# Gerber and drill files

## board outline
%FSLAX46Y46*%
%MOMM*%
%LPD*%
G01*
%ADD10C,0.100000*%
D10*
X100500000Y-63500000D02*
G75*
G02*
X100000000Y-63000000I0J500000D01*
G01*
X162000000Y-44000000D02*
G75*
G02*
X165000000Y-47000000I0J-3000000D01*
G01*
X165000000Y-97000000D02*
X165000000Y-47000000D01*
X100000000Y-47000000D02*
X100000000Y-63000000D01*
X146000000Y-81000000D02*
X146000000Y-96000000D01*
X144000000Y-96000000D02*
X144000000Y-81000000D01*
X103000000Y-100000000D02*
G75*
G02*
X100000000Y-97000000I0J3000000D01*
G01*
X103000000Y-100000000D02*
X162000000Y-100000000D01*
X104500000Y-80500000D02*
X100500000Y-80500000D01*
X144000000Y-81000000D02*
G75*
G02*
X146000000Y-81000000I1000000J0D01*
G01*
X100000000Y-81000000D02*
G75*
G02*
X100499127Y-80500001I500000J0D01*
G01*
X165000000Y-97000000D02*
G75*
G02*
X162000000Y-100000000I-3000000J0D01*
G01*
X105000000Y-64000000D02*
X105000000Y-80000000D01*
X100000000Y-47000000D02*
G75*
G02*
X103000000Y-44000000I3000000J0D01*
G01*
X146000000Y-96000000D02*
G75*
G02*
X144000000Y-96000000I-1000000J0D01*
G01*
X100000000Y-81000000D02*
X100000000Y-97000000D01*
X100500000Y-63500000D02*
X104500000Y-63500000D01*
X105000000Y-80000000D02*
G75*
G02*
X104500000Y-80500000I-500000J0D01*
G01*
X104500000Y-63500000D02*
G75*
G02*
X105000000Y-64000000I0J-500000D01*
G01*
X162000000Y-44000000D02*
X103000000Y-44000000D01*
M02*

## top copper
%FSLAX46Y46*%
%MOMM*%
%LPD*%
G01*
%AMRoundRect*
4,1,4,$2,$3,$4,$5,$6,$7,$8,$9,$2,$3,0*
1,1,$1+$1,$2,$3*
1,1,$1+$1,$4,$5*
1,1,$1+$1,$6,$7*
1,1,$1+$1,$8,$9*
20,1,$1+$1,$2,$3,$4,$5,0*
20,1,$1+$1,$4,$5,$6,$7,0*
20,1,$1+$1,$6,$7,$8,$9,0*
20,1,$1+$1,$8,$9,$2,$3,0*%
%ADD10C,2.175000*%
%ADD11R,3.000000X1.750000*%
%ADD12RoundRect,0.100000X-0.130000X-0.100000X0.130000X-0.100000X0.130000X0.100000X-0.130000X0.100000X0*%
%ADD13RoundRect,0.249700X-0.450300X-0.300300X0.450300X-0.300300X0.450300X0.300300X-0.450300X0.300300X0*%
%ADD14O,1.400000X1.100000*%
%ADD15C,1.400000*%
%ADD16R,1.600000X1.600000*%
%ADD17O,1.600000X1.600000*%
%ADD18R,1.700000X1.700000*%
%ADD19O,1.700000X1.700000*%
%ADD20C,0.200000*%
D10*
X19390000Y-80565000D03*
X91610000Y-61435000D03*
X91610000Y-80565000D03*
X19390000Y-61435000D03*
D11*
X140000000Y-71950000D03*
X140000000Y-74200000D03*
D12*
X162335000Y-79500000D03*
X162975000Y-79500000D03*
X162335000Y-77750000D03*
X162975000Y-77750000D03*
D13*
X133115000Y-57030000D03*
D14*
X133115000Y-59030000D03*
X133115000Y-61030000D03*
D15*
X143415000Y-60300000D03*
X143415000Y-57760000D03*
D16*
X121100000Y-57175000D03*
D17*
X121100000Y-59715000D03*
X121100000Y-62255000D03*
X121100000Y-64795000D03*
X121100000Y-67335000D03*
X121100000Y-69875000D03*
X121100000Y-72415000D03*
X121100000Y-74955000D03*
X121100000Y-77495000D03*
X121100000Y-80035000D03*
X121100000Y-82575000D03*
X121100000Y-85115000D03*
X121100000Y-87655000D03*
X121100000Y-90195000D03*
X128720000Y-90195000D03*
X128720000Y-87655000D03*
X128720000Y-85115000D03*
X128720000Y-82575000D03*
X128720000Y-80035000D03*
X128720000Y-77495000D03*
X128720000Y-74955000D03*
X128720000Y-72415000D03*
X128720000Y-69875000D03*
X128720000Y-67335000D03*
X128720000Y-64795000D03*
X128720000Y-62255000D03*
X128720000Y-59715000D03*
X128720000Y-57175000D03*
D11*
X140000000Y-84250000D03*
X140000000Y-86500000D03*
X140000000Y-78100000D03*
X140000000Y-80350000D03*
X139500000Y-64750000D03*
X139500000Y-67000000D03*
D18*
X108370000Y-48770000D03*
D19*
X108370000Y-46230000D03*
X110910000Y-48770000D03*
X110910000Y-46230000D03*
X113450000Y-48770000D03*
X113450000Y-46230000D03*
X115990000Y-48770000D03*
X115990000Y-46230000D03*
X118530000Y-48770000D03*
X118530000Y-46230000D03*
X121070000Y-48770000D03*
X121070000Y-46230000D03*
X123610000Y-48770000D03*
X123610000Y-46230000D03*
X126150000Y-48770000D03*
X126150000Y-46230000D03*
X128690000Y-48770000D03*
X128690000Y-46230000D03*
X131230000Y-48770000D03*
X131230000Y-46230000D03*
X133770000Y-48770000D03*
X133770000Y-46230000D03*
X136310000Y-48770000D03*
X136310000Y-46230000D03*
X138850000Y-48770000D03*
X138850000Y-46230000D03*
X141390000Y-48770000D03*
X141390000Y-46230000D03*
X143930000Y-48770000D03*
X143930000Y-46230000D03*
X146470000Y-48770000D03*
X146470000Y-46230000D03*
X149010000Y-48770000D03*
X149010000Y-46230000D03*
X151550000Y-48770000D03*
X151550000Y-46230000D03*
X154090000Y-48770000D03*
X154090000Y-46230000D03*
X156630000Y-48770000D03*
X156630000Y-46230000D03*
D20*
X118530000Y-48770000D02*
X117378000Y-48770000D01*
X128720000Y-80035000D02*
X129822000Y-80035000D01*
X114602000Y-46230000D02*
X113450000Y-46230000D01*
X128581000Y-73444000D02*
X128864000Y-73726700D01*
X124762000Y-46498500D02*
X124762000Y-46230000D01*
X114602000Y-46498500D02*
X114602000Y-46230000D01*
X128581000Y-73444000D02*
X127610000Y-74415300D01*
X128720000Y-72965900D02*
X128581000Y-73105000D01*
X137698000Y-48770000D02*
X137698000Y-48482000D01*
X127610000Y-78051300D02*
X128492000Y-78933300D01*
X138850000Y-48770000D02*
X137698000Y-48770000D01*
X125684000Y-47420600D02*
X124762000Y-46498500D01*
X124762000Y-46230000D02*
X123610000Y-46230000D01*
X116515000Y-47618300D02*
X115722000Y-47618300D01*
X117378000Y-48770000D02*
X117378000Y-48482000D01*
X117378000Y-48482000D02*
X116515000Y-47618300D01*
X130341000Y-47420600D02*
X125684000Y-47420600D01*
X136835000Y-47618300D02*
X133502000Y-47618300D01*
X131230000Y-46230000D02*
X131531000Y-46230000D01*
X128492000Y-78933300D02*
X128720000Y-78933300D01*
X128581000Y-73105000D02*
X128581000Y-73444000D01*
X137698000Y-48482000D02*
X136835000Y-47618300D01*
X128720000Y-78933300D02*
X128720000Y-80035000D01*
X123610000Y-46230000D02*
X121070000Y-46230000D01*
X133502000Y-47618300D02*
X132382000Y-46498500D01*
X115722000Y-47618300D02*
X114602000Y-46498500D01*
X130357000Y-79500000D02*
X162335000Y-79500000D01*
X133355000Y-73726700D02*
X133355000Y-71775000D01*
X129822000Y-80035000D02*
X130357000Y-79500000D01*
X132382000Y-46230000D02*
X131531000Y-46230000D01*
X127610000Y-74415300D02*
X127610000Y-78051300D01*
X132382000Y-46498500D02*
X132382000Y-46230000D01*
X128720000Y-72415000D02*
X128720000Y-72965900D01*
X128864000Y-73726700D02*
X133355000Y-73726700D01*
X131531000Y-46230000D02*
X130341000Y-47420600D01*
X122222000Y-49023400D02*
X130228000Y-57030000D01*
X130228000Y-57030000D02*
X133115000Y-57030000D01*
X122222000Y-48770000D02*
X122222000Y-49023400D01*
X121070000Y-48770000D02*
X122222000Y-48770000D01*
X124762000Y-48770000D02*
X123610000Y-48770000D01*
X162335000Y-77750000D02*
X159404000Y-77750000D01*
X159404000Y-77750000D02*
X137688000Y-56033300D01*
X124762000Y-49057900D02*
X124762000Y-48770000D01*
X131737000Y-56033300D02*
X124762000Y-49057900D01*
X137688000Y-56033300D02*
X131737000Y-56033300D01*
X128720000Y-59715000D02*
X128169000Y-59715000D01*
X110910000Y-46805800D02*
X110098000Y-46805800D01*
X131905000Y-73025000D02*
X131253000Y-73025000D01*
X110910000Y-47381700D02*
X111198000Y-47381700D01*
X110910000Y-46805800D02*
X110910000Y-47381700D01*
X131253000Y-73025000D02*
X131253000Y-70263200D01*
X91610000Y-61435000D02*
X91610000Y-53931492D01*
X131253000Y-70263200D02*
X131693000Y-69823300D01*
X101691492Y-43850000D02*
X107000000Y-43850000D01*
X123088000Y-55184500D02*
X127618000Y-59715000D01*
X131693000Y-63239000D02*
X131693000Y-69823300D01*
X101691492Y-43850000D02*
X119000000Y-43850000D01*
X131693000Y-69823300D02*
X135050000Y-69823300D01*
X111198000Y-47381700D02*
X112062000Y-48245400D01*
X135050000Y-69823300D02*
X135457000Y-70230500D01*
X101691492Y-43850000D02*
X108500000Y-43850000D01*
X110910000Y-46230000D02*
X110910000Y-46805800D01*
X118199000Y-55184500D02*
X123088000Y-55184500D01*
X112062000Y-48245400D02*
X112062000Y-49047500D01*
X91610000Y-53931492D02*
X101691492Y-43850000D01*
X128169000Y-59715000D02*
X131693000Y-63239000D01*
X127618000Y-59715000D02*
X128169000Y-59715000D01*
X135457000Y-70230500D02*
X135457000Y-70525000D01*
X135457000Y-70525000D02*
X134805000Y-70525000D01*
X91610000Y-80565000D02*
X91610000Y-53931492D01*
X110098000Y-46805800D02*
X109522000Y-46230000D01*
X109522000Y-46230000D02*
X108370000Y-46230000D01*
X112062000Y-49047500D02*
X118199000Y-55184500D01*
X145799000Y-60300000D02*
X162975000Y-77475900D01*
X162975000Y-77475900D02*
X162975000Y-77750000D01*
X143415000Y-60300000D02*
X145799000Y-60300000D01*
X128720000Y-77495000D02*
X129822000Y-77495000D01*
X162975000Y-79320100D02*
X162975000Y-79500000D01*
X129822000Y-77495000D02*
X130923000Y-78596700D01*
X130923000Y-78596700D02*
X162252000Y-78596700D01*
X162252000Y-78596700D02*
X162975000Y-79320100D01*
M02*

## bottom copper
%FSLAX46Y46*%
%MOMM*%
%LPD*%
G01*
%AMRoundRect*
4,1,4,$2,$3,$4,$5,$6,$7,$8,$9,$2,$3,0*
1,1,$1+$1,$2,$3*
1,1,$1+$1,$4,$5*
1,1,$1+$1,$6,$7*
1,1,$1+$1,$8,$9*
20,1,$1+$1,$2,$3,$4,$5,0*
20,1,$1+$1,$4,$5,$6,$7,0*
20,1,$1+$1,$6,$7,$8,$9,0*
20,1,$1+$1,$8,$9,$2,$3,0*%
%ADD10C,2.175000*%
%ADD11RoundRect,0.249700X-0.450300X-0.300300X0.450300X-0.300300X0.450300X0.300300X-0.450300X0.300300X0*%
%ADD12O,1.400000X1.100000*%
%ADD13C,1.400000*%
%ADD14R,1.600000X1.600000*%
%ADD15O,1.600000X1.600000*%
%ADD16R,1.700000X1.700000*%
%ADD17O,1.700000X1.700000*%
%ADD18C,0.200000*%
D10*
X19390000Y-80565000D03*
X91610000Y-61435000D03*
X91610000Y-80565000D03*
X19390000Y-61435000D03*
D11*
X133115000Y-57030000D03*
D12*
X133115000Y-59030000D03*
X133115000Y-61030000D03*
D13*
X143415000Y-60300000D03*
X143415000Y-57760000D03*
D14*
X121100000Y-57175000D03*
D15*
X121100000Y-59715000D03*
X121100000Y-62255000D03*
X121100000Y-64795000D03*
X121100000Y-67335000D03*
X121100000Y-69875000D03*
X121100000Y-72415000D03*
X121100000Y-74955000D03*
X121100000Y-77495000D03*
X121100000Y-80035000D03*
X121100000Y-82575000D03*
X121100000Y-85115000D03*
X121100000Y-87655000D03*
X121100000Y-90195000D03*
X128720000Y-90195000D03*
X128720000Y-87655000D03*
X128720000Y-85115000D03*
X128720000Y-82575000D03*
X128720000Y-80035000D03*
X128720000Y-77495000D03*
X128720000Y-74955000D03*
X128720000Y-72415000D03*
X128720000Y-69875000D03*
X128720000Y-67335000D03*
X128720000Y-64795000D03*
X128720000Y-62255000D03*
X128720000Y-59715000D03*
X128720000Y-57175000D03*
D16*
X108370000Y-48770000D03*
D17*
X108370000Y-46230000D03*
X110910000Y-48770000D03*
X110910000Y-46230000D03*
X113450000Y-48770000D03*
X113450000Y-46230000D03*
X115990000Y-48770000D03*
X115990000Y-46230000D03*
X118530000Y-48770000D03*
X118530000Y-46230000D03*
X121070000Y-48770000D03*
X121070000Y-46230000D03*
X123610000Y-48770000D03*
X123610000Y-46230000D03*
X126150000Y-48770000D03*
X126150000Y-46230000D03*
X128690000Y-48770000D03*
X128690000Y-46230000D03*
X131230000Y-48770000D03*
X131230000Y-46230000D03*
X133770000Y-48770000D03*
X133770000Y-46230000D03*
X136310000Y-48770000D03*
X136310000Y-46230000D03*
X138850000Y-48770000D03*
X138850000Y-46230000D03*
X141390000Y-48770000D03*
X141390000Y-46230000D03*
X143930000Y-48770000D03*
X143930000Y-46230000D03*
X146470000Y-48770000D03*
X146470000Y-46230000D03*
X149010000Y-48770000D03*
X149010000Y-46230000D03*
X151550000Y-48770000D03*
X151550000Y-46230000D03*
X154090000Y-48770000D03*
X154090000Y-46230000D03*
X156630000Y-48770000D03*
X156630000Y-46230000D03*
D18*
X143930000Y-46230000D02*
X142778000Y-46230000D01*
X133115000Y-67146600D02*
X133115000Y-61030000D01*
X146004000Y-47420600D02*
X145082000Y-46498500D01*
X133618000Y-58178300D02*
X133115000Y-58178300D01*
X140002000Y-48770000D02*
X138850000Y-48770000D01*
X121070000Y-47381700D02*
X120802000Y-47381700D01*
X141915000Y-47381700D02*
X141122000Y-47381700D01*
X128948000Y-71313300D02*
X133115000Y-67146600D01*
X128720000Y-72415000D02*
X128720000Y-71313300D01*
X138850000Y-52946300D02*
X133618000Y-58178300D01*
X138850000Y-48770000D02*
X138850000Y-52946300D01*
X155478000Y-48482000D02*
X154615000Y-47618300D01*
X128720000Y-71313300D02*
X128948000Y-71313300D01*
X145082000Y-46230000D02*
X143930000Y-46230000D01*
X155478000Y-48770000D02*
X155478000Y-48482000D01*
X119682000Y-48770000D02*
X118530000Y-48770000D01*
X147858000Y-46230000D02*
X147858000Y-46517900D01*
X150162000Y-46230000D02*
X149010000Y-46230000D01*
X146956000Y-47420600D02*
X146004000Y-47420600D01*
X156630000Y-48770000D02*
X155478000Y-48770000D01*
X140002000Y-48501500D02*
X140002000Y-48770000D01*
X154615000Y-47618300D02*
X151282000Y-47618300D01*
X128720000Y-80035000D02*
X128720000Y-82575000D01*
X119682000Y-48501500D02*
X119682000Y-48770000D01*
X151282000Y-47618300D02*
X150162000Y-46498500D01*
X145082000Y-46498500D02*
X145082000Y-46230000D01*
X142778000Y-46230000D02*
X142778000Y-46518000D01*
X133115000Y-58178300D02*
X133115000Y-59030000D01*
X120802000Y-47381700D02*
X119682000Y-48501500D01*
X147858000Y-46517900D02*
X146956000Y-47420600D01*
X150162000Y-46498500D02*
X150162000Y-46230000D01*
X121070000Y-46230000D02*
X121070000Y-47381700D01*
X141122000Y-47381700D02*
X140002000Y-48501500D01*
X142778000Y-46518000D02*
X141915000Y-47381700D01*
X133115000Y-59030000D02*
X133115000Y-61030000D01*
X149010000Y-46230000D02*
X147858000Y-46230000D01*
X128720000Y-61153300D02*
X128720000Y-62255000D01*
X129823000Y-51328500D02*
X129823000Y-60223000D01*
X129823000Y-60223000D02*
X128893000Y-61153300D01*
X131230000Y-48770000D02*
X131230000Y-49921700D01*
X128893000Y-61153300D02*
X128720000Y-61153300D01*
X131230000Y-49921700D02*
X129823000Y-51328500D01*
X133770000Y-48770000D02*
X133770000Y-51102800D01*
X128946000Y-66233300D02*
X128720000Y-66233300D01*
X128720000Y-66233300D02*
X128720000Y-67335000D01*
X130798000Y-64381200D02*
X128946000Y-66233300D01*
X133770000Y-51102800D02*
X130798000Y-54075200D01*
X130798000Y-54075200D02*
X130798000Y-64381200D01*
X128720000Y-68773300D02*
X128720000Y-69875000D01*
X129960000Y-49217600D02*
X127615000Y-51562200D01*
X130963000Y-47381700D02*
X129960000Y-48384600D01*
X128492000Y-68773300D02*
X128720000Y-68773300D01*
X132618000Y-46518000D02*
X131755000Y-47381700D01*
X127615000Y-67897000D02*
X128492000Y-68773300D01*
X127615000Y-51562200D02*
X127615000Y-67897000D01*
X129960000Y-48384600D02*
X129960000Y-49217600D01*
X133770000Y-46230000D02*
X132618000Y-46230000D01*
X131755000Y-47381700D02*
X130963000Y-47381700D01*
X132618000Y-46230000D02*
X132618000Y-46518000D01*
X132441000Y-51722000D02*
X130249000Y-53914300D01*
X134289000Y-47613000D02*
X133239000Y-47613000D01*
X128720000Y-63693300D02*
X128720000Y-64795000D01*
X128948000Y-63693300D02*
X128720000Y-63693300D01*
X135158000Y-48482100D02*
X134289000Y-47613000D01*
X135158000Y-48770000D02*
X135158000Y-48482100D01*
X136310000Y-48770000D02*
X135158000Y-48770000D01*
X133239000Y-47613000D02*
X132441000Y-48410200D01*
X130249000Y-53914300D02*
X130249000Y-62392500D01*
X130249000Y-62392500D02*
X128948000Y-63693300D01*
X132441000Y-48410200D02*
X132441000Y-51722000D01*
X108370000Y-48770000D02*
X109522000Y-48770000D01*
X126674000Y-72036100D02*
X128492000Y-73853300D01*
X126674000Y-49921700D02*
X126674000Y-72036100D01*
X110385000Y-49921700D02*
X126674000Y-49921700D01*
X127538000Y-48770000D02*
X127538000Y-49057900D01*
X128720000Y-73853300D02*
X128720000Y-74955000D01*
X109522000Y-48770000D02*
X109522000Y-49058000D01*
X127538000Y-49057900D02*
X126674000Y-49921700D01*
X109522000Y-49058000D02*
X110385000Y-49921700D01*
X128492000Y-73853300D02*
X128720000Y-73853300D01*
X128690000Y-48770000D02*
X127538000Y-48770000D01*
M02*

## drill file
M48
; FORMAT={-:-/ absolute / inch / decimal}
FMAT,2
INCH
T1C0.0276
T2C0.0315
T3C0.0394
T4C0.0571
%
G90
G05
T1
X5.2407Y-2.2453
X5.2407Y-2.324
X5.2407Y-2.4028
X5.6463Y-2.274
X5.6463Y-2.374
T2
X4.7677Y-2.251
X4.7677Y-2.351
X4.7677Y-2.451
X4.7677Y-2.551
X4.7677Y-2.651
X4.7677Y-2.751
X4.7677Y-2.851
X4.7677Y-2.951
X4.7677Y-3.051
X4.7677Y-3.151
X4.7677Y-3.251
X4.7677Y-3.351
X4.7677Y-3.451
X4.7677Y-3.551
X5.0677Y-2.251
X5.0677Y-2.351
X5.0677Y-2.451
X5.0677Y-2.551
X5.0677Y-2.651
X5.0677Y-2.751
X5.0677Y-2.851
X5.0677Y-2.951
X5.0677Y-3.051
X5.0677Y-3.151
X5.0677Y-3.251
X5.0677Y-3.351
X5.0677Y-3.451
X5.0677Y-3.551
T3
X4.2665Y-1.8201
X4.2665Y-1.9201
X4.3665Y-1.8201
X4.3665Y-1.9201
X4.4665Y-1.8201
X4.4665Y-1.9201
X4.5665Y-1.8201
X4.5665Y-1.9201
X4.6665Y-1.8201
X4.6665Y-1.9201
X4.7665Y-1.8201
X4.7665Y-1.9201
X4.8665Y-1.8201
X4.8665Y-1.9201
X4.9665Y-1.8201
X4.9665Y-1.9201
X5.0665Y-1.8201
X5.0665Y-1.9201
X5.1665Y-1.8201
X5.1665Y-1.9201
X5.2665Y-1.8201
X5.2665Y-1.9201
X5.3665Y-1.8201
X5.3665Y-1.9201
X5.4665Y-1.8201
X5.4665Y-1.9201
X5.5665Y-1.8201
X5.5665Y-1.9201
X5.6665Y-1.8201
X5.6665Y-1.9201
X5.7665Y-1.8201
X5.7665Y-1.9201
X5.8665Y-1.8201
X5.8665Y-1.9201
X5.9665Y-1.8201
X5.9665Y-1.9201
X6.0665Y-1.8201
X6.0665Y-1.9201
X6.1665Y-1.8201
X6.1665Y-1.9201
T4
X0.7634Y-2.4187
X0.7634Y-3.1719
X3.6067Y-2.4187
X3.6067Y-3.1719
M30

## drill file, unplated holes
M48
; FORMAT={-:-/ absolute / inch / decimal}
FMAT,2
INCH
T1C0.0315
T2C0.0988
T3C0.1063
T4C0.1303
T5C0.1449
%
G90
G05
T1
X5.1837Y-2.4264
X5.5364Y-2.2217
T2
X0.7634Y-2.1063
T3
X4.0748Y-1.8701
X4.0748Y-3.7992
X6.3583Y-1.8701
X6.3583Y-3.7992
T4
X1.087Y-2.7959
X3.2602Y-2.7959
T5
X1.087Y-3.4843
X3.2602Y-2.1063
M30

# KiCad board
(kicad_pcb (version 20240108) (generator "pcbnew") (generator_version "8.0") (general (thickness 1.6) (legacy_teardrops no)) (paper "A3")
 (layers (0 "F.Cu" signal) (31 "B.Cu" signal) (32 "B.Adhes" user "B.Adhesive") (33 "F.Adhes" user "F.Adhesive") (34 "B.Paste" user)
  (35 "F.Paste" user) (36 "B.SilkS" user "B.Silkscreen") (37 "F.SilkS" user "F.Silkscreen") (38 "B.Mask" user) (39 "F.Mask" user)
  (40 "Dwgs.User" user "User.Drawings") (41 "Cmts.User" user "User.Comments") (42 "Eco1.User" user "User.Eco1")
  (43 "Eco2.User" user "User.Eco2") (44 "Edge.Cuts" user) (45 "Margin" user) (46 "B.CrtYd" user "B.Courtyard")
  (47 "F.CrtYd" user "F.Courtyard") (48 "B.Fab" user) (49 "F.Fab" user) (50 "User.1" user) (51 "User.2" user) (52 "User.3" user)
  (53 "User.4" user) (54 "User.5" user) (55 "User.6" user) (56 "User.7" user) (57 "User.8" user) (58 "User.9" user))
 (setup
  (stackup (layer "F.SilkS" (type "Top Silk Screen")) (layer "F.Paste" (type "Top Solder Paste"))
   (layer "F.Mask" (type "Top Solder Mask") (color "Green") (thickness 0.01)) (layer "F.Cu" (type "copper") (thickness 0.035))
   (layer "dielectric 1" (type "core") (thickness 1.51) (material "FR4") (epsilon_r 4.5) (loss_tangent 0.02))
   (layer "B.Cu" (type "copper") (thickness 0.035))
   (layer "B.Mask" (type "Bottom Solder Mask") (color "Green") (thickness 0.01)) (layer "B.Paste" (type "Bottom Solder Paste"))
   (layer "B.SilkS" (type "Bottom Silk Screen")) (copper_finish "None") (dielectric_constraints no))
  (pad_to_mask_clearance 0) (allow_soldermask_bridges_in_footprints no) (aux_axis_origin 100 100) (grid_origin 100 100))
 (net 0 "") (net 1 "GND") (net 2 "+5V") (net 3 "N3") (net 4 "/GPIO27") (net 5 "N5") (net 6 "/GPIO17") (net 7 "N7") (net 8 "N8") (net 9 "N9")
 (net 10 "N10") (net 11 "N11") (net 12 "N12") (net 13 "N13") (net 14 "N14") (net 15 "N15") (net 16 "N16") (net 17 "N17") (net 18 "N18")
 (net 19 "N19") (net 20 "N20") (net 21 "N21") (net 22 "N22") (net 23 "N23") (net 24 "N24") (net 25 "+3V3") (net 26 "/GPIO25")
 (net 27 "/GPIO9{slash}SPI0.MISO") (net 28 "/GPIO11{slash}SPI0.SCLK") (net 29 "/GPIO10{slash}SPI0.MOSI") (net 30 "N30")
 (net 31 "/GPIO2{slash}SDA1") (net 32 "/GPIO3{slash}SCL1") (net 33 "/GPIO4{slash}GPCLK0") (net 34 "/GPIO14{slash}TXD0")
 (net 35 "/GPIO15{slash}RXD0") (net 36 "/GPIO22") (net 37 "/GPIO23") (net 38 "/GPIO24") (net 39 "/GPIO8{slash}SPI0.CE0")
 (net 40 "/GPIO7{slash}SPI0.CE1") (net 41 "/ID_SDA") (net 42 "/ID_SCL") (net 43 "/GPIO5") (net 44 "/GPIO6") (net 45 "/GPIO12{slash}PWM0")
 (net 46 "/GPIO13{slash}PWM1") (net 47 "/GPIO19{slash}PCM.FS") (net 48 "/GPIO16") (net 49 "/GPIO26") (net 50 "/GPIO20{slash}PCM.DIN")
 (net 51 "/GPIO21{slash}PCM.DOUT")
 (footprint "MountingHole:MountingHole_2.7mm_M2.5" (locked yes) (layer "F.Cu") (at 161.5 47.5)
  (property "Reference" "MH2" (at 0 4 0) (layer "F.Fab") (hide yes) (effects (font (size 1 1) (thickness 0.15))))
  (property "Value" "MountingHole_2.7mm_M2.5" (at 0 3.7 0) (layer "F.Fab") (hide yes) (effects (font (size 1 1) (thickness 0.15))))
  (pad "" np_thru_hole circle (at 0 0) (size 2.7 2.7) (drill 2.7) (layers "*.Cu" "*.Mask")))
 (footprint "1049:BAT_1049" (layer "F.Cu") (at 55.5 71 180)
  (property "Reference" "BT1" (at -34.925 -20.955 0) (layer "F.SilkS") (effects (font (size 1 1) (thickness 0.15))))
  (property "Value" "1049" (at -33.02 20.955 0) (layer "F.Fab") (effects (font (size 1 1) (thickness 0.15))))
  (pad "" np_thru_hole circle (at -27.31 -0.015 180) (size 3.31 3.31) (drill 3.31) (layers "*.Cu" "*.Mask"))
  (pad "" np_thru_hole circle (at -27.31 17.5 180) (size 3.68 3.68) (drill 3.68) (layers "*.Cu" "*.Mask"))
  (pad "" np_thru_hole circle (at 27.89 -17.5 180) (size 3.68 3.68) (drill 3.68) (layers "*.Cu" "*.Mask"))
  (pad "" np_thru_hole circle (at 27.89 -0.015 180) (size 3.31 3.31) (drill 3.31) (layers "*.Cu" "*.Mask"))
  (pad "" np_thru_hole circle (at 36.11 17.5 180) (size 2.51 2.51) (drill 2.51) (layers "*.Cu" "*.Mask"))
  (pad "N1" thru_hole circle (at 36.11 -9.565 180) (size 2.175 2.175) (drill 1.45) (layers "*.Cu" "*.Mask") (remove_unused_layers no)
   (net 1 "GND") (solder_mask_margin 0.102))
  (pad "N2" thru_hole circle (at -36.11 9.565 180) (size 2.175 2.175) (drill 1.45) (layers "*.Cu" "*.Mask") (remove_unused_layers no)
   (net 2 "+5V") (solder_mask_margin 0.102))
  (pad "P1" thru_hole circle (at -36.11 -9.565 180) (size 2.175 2.175) (drill 1.45) (layers "*.Cu" "*.Mask") (remove_unused_layers no)
   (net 2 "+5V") (solder_mask_margin 0.102))
  (pad "P2" thru_hole circle (at 36.11 9.565 180) (size 2.175 2.175) (drill 1.45) (layers "*.Cu" "*.Mask") (remove_unused_layers no)
   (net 1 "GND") (solder_mask_margin 0.102)))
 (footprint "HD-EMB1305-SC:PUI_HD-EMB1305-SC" (layer "F.Cu") (at 140 73.075)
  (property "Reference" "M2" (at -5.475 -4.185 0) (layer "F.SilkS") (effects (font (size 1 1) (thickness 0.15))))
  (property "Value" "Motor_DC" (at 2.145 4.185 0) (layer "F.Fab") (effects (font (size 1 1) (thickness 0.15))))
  (pad "N" smd rect (at 0 -1.125) (size 3 1.75) (layers "F.Cu" "F.Paste" "F.Mask") (solder_mask_margin 0.102))
  (pad "P" smd rect (at 0 1.125) (size 3 1.75) (layers "F.Cu" "F.Paste" "F.Mask") (solder_mask_margin 0.102)))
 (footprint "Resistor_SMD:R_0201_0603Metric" (layer "F.Cu") (at 162.655 79.5)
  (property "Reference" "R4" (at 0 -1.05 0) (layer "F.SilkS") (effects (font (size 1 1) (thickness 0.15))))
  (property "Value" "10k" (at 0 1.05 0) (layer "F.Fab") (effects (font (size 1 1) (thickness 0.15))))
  (pad "" smd roundrect (at -0.345 0) (size 0.318 0.36) (layers "F.Paste") (roundrect_rratio 0.25))
  (pad "" smd roundrect (at 0.345 0) (size 0.318 0.36) (layers "F.Paste") (roundrect_rratio 0.25))
  (pad "1" smd roundrect (at -0.32 0) (size 0.46 0.4) (layers "F.Cu" "F.Mask") (roundrect_rratio 0.25) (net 1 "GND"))
  (pad "2" smd roundrect (at 0.32 0) (size 0.46 0.4) (layers "F.Cu" "F.Mask") (roundrect_rratio 0.25) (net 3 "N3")))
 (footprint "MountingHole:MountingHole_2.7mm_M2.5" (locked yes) (layer "F.Cu") (at 103.5 96.5)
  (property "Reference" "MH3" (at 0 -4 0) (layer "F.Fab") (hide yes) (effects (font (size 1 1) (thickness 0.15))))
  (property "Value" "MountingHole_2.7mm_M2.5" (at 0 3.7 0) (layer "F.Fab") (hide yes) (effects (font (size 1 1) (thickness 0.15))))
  (pad "" np_thru_hole circle (at 0 0) (size 2.7 2.7) (drill 2.7) (layers "*.Cu" "*.Mask")))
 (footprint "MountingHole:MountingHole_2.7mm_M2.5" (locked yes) (layer "F.Cu") (at 103.5 47.5)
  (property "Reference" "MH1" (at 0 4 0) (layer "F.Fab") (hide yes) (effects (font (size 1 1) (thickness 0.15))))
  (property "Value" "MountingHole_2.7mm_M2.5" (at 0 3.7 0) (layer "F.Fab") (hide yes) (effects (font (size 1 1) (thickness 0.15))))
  (pad "" np_thru_hole circle (at 0 0) (size 2.7 2.7) (drill 2.7) (layers "*.Cu" "*.Mask")))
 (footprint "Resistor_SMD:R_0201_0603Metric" (layer "F.Cu") (at 162.655 77.75)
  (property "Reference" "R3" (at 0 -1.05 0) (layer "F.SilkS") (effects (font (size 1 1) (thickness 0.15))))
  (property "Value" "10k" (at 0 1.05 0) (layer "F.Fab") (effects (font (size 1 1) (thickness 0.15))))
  (pad "" smd roundrect (at -0.345 0) (size 0.318 0.36) (layers "F.Paste") (roundrect_rratio 0.25))
  (pad "" smd roundrect (at 0.345 0) (size 0.318 0.36) (layers "F.Paste") (roundrect_rratio 0.25))
  (pad "1" smd roundrect (at -0.32 0) (size 0.46 0.4) (layers "F.Cu" "F.Mask") (roundrect_rratio 0.25) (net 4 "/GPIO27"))
  (pad "2" smd roundrect (at 0.32 0) (size 0.46 0.4) (layers "F.Cu" "F.Mask") (roundrect_rratio 0.25) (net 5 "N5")))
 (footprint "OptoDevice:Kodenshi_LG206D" (layer "F.Cu") (at 133.115 57.03)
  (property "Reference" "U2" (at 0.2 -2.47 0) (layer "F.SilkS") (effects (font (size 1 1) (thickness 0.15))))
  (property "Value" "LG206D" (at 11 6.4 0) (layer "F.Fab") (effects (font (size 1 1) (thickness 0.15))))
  (pad "" np_thru_hole circle (at -1.45 4.6) (size 0.8 0.8) (drill 0.8) (layers "*.Cu" "*.Mask"))
  (pad "" np_thru_hole circle (at 7.51 -0.6) (size 0.8 0.8) (drill 0.8) (layers "*.Cu" "*.Mask"))
  (pad "1" thru_hole roundrect (at 0 0) (size 1.4 1.1) (drill 0.7) (layers "*.Cu" "*.Mask") (remove_unused_layers no)
   (roundrect_rratio 0.227) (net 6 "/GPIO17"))
  (pad "2" thru_hole oval (at 0 2) (size 1.4 1.1) (drill 0.7) (layers "*.Cu" "*.Mask") (remove_unused_layers no) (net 1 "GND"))
  (pad "3" thru_hole oval (at 0 4) (size 1.4 1.1) (drill 0.7) (layers "*.Cu" "*.Mask") (remove_unused_layers no) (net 1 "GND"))
  (pad "4" thru_hole circle (at 10.3 3.27) (size 1.4 1.4) (drill 0.7) (layers "*.Cu" "*.Mask") (remove_unused_layers no) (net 5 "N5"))
  (pad "5" thru_hole circle (at 10.3 0.73) (size 1.4 1.4) (drill 0.7) (layers "*.Cu" "*.Mask") (remove_unused_layers no) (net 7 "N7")))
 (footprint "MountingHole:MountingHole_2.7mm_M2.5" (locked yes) (layer "F.Cu") (at 161.5 96.5)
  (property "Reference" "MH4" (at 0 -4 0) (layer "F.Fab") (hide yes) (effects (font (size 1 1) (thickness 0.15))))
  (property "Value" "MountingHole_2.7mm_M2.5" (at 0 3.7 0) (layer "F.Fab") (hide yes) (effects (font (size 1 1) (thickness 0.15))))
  (pad "" np_thru_hole circle (at 0 0) (size 2.7 2.7) (drill 2.7) (layers "*.Cu" "*.Mask")))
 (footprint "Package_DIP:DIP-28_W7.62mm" (layer "F.Cu") (at 121.1 57.175)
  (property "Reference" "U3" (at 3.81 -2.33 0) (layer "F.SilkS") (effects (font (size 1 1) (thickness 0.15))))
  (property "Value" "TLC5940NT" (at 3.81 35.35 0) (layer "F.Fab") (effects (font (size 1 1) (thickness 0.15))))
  (pad "1" thru_hole rect (at 0 0) (size 1.6 1.6) (drill 0.8) (layers "*.Cu" "*.Mask") (remove_unused_layers no) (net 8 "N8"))
  (pad "2" thru_hole oval (at 0 2.54) (size 1.6 1.6) (drill 0.8) (layers "*.Cu" "*.Mask") (remove_unused_layers no) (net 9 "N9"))
  (pad "3" thru_hole oval (at 0 5.08) (size 1.6 1.6) (drill 0.8) (layers "*.Cu" "*.Mask") (remove_unused_layers no) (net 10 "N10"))
  (pad "4" thru_hole oval (at 0 7.62) (size 1.6 1.6) (drill 0.8) (layers "*.Cu" "*.Mask") (remove_unused_layers no) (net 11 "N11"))
  (pad "5" thru_hole oval (at 0 10.16) (size 1.6 1.6) (drill 0.8) (layers "*.Cu" "*.Mask") (remove_unused_layers no) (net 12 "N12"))
  (pad "6" thru_hole oval (at 0 12.7) (size 1.6 1.6) (drill 0.8) (layers "*.Cu" "*.Mask") (remove_unused_layers no) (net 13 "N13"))
  (pad "7" thru_hole oval (at 0 15.24) (size 1.6 1.6) (drill 0.8) (layers "*.Cu" "*.Mask") (remove_unused_layers no) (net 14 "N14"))
  (pad "8" thru_hole oval (at 0 17.78) (size 1.6 1.6) (drill 0.8) (layers "*.Cu" "*.Mask") (remove_unused_layers no) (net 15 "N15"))
  (pad "9" thru_hole oval (at 0 20.32) (size 1.6 1.6) (drill 0.8) (layers "*.Cu" "*.Mask") (remove_unused_layers no) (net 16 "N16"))
  (pad "10" thru_hole oval (at 0 22.86) (size 1.6 1.6) (drill 0.8) (layers "*.Cu" "*.Mask") (remove_unused_layers no) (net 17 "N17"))
  (pad "11" thru_hole oval (at 0 25.4) (size 1.6 1.6) (drill 0.8) (layers "*.Cu" "*.Mask") (remove_unused_layers no) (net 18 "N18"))
  (pad "12" thru_hole oval (at 0 27.94) (size 1.6 1.6) (drill 0.8) (layers "*.Cu" "*.Mask") (remove_unused_layers no) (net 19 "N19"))
  (pad "13" thru_hole oval (at 0 30.48) (size 1.6 1.6) (drill 0.8) (layers "*.Cu" "*.Mask") (remove_unused_layers no) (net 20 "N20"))
  (pad "14" thru_hole oval (at 0 33.02) (size 1.6 1.6) (drill 0.8) (layers "*.Cu" "*.Mask") (remove_unused_layers no) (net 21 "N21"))
  (pad "15" thru_hole oval (at 7.62 33.02) (size 1.6 1.6) (drill 0.8) (layers "*.Cu" "*.Mask") (remove_unused_layers no) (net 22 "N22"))
  (pad "16" thru_hole oval (at 7.62 30.48) (size 1.6 1.6) (drill 0.8) (layers "*.Cu" "*.Mask") (remove_unused_layers no) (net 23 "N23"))
  (pad "17" thru_hole oval (at 7.62 27.94) (size 1.6 1.6) (drill 0.8) (layers "*.Cu" "*.Mask") (remove_unused_layers no) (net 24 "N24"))
  (pad "18" thru_hole oval (at 7.62 25.4) (size 1.6 1.6) (drill 0.8) (layers "*.Cu" "*.Mask") (remove_unused_layers no) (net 1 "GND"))
  (pad "19" thru_hole oval (at 7.62 22.86) (size 1.6 1.6) (drill 0.8) (layers "*.Cu" "*.Mask") (remove_unused_layers no) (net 1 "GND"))
  (pad "20" thru_hole oval (at 7.62 20.32) (size 1.6 1.6) (drill 0.8) (layers "*.Cu" "*.Mask") (remove_unused_layers no) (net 3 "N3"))
  (pad "21" thru_hole oval (at 7.62 17.78) (size 1.6 1.6) (drill 0.8) (layers "*.Cu" "*.Mask") (remove_unused_layers no) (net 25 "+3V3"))
  (pad "22" thru_hole oval (at 7.62 15.24) (size 1.6 1.6) (drill 0.8) (layers "*.Cu" "*.Mask") (remove_unused_layers no) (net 1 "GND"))
  (pad "23" thru_hole oval (at 7.62 12.7) (size 1.6 1.6) (drill 0.8) (layers "*.Cu" "*.Mask") (remove_unused_layers no) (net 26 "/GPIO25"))
  (pad "24" thru_hole oval (at 7.62 10.16) (size 1.6 1.6) (drill 0.8) (layers "*.Cu" "*.Mask") (remove_unused_layers no)
   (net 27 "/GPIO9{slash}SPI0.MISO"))
  (pad "25" thru_hole oval (at 7.62 7.62) (size 1.6 1.6) (drill 0.8) (layers "*.Cu" "*.Mask") (remove_unused_layers no)
   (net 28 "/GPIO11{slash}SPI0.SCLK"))
  (pad "26" thru_hole oval (at 7.62 5.08) (size 1.6 1.6) (drill 0.8) (layers "*.Cu" "*.Mask") (remove_unused_layers no)
   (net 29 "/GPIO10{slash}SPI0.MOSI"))
  (pad "27" thru_hole oval (at 7.62 2.54) (size 1.6 1.6) (drill 0.8) (layers "*.Cu" "*.Mask") (remove_unused_layers no) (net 2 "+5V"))
  (pad "28" thru_hole oval (at 7.62 0) (size 1.6 1.6) (drill 0.8) (layers "*.Cu" "*.Mask") (remove_unused_layers no) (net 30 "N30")))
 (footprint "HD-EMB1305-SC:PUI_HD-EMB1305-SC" (layer "F.Cu") (at 140 85.375)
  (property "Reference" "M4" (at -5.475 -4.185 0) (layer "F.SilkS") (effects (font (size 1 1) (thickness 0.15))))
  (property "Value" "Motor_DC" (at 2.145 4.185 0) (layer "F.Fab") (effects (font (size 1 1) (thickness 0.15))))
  (pad "N" smd rect (at 0 -1.125) (size 3 1.75) (layers "F.Cu" "F.Paste" "F.Mask") (solder_mask_margin 0.102))
  (pad "P" smd rect (at 0 1.125) (size 3 1.75) (layers "F.Cu" "F.Paste" "F.Mask") (solder_mask_margin 0.102)))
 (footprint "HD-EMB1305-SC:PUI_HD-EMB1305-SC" (layer "F.Cu") (at 140 79.225)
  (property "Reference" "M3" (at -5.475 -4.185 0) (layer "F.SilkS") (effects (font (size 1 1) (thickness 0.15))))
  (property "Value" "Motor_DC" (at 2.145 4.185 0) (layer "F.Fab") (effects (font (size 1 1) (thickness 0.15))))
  (pad "N" smd rect (at 0 -1.125) (size 3 1.75) (layers "F.Cu" "F.Paste" "F.Mask") (solder_mask_margin 0.102))
  (pad "P" smd rect (at 0 1.125) (size 3 1.75) (layers "F.Cu" "F.Paste" "F.Mask") (solder_mask_margin 0.102)))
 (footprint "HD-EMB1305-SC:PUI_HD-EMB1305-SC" (layer "F.Cu") (at 139.5 65.875)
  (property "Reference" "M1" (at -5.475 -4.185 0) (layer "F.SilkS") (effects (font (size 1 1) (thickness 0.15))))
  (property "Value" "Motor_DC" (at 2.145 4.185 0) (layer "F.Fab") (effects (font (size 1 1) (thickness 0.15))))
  (pad "N" smd rect (at 0 -1.125) (size 3 1.75) (layers "F.Cu" "F.Paste" "F.Mask") (solder_mask_margin 0.102))
  (pad "P" smd rect (at 0 1.125) (size 3 1.75) (layers "F.Cu" "F.Paste" "F.Mask") (solder_mask_margin 0.102)))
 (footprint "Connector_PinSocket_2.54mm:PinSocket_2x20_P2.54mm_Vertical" (layer "B.Cu") (at 108.37 48.77 -90)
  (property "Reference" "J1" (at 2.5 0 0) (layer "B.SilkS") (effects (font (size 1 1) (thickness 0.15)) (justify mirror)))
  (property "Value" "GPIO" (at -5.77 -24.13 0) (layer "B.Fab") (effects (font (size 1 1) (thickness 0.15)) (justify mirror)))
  (pad "1" thru_hole rect (at 0 0 270) (size 1.7 1.7) (drill 1) (layers "*.Cu" "*.Mask") (remove_unused_layers no) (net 25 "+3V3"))
  (pad "2" thru_hole oval (at -2.54 0 270) (size 1.7 1.7) (drill 1) (layers "*.Cu" "*.Mask") (remove_unused_layers no) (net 2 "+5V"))
  (pad "3" thru_hole oval (at 0 -2.54 270) (size 1.7 1.7) (drill 1) (layers "*.Cu" "*.Mask") (remove_unused_layers no)
   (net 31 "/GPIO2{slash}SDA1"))
  (pad "4" thru_hole oval (at -2.54 -2.54 270) (size 1.7 1.7) (drill 1) (layers "*.Cu" "*.Mask") (remove_unused_layers no) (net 2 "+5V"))
  (pad "5" thru_hole oval (at 0 -5.08 270) (size 1.7 1.7) (drill 1) (layers "*.Cu" "*.Mask") (remove_unused_layers no)
   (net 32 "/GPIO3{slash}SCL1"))
  (pad "6" thru_hole oval (at -2.54 -5.08 270) (size 1.7 1.7) (drill 1) (layers "*.Cu" "*.Mask") (remove_unused_layers no) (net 1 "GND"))
  (pad "7" thru_hole oval (at 0 -7.62 270) (size 1.7 1.7) (drill 1) (layers "*.Cu" "*.Mask") (remove_unused_layers no)
   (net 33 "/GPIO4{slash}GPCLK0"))
  (pad "8" thru_hole oval (at -2.54 -7.62 270) (size 1.7 1.7) (drill 1) (layers "*.Cu" "*.Mask") (remove_unused_layers no)
   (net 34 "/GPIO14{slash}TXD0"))
  (pad "9" thru_hole oval (at 0 -10.16 270) (size 1.7 1.7) (drill 1) (layers "*.Cu" "*.Mask") (remove_unused_layers no) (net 1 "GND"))
  (pad "10" thru_hole oval (at -2.54 -10.16 270) (size 1.7 1.7) (drill 1) (layers "*.Cu" "*.Mask") (remove_unused_layers no)
   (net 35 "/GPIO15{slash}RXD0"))
  (pad "11" thru_hole oval (at 0 -12.7 270) (size 1.7 1.7) (drill 1) (layers "*.Cu" "*.Mask") (remove_unused_layers no) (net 6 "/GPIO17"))
  (pad "12" thru_hole oval (at -2.54 -12.7 270) (size 1.7 1.7) (drill 1) (layers "*.Cu" "*.Mask") (remove_unused_layers no) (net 1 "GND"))
  (pad "13" thru_hole oval (at 0 -15.24 270) (size 1.7 1.7) (drill 1) (layers "*.Cu" "*.Mask") (remove_unused_layers no) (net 4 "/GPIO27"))
  (pad "14" thru_hole oval (at -2.54 -15.24 270) (size 1.7 1.7) (drill 1) (layers "*.Cu" "*.Mask") (remove_unused_layers no) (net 1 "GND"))
  (pad "15" thru_hole oval (at 0 -17.78 270) (size 1.7 1.7) (drill 1) (layers "*.Cu" "*.Mask") (remove_unused_layers no) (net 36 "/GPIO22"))
  (pad "16" thru_hole oval (at -2.54 -17.78 270) (size 1.7 1.7) (drill 1) (layers "*.Cu" "*.Mask") (remove_unused_layers no)
   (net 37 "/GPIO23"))
  (pad "17" thru_hole oval (at 0 -20.32 270) (size 1.7 1.7) (drill 1) (layers "*.Cu" "*.Mask") (remove_unused_layers no) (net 25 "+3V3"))
  (pad "18" thru_hole oval (at -2.54 -20.32 270) (size 1.7 1.7) (drill 1) (layers "*.Cu" "*.Mask") (remove_unused_layers no)
   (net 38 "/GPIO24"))
  (pad "19" thru_hole oval (at 0 -22.86 270) (size 1.7 1.7) (drill 1) (layers "*.Cu" "*.Mask") (remove_unused_layers no)
   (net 29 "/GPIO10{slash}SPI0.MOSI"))
  (pad "20" thru_hole oval (at -2.54 -22.86 270) (size 1.7 1.7) (drill 1) (layers "*.Cu" "*.Mask") (remove_unused_layers no) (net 1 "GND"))
  (pad "21" thru_hole oval (at 0 -25.4 270) (size 1.7 1.7) (drill 1) (layers "*.Cu" "*.Mask") (remove_unused_layers no)
   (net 27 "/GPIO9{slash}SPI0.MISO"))
  (pad "22" thru_hole oval (at -2.54 -25.4 270) (size 1.7 1.7) (drill 1) (layers "*.Cu" "*.Mask") (remove_unused_layers no)
   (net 26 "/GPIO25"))
  (pad "23" thru_hole oval (at 0 -27.94 270) (size 1.7 1.7) (drill 1) (layers "*.Cu" "*.Mask") (remove_unused_layers no)
   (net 28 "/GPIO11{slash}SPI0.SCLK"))
  (pad "24" thru_hole oval (at -2.54 -27.94 270) (size 1.7 1.7) (drill 1) (layers "*.Cu" "*.Mask") (remove_unused_layers no)
   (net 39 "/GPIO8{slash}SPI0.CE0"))
  (pad "25" thru_hole oval (at 0 -30.48 270) (size 1.7 1.7) (drill 1) (layers "*.Cu" "*.Mask") (remove_unused_layers no) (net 1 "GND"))
  (pad "26" thru_hole oval (at -2.54 -30.48 270) (size 1.7 1.7) (drill 1) (layers "*.Cu" "*.Mask") (remove_unused_layers no)
   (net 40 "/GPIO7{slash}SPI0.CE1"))
  (pad "27" thru_hole oval (at 0 -33.02 270) (size 1.7 1.7) (drill 1) (layers "*.Cu" "*.Mask") (remove_unused_layers no) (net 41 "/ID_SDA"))
  (pad "28" thru_hole oval (at -2.54 -33.02 270) (size 1.7 1.7) (drill 1) (layers "*.Cu" "*.Mask") (remove_unused_layers no)
   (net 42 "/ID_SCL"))
  (pad "29" thru_hole oval (at 0 -35.56 270) (size 1.7 1.7) (drill 1) (layers "*.Cu" "*.Mask") (remove_unused_layers no) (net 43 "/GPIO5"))
  (pad "30" thru_hole oval (at -2.54 -35.56 270) (size 1.7 1.7) (drill 1) (layers "*.Cu" "*.Mask") (remove_unused_layers no) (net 1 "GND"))
  (pad "31" thru_hole oval (at 0 -38.1 270) (size 1.7 1.7) (drill 1) (layers "*.Cu" "*.Mask") (remove_unused_layers no) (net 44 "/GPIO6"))
  (pad "32" thru_hole oval (at -2.54 -38.1 270) (size 1.7 1.7) (drill 1) (layers "*.Cu" "*.Mask") (remove_unused_layers no)
   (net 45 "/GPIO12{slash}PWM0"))
  (pad "33" thru_hole oval (at 0 -40.64 270) (size 1.7 1.7) (drill 1) (layers "*.Cu" "*.Mask") (remove_unused_layers no)
   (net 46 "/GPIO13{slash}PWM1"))
  (pad "34" thru_hole oval (at -2.54 -40.64 270) (size 1.7 1.7) (drill 1) (layers "*.Cu" "*.Mask") (remove_unused_layers no) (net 1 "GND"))
  (pad "35" thru_hole oval (at 0 -43.18 270) (size 1.7 1.7) (drill 1) (layers "*.Cu" "*.Mask") (remove_unused_layers no)
   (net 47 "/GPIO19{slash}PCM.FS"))
  (pad "36" thru_hole oval (at -2.54 -43.18 270) (size 1.7 1.7) (drill 1) (layers "*.Cu" "*.Mask") (remove_unused_layers no)
   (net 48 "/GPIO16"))
  (pad "37" thru_hole oval (at 0 -45.72 270) (size 1.7 1.7) (drill 1) (layers "*.Cu" "*.Mask") (remove_unused_layers no) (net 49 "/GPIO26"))
  (pad "38" thru_hole oval (at -2.54 -45.72 270) (size 1.7 1.7) (drill 1) (layers "*.Cu" "*.Mask") (remove_unused_layers no)
   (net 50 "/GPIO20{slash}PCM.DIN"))
  (pad "39" thru_hole oval (at 0 -48.26 270) (size 1.7 1.7) (drill 1) (layers "*.Cu" "*.Mask") (remove_unused_layers no) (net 1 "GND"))
  (pad "40" thru_hole oval (at -2.54 -48.26 270) (size 1.7 1.7) (drill 1) (layers "*.Cu" "*.Mask") (remove_unused_layers no)
   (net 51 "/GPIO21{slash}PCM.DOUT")))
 (gr_arc (start 100.5 63.5) (mid 100.146447 63.353553) (end 100 63) (stroke (width 0.1) (type solid)) (layer "Edge.Cuts"))
 (gr_arc (start 162 44) (mid 164.12132 44.87868) (end 165 47) (stroke (width 0.1) (type solid)) (layer "Edge.Cuts"))
 (gr_line (start 165 97) (end 165 47) (stroke (width 0.1) (type solid)) (layer "Edge.Cuts"))
 (gr_line (start 100 47) (end 100 63) (stroke (width 0.1) (type solid)) (layer "Edge.Cuts"))
 (gr_line (start 146 81) (end 146 96) (stroke (width 0.1) (type solid)) (layer "Edge.Cuts"))
 (gr_line (start 144 96) (end 144 81) (stroke (width 0.1) (type solid)) (layer "Edge.Cuts"))
 (gr_arc (start 103 100) (mid 100.87868 99.12132) (end 100 97) (stroke (width 0.1) (type solid)) (layer "Edge.Cuts"))
 (gr_line (start 103 100) (end 162 100) (stroke (width 0.1) (type solid)) (layer "Edge.Cuts"))
 (gr_line (start 104.5 80.5) (end 100.5 80.5) (stroke (width 0.1) (type solid)) (layer "Edge.Cuts"))
 (gr_arc (start 144 81) (mid 145 80) (end 146 81) (stroke (width 0.1) (type solid)) (layer "Edge.Cuts"))
 (gr_arc (start 100 81) (mid 100.146138 80.646755) (end 100.499127 80.500001) (stroke (width 0.1) (type solid)) (layer "Edge.Cuts"))
 (gr_arc (start 165 97) (mid 164.12132 99.12132) (end 162 100) (stroke (width 0.1) (type solid)) (layer "Edge.Cuts"))
 (gr_line (start 105 64) (end 105 80) (stroke (width 0.1) (type solid)) (layer "Edge.Cuts"))
 (gr_arc (start 100 47) (mid 100.87868 44.87868) (end 103 44) (stroke (width 0.1) (type solid)) (layer "Edge.Cuts"))
 (gr_arc (start 146 96) (mid 145 97) (end 144 96) (stroke (width 0.1) (type solid)) (layer "Edge.Cuts"))
 (gr_line (start 100 81) (end 100 97) (stroke (width 0.1) (type solid)) (layer "Edge.Cuts"))
 (gr_line (start 100.5 63.5) (end 104.5 63.5) (stroke (width 0.1) (type solid)) (layer "Edge.Cuts"))
 (gr_arc (start 105 80) (mid 104.853553 80.353553) (end 104.5 80.5) (stroke (width 0.1) (type solid)) (layer "Edge.Cuts"))
 (gr_arc (start 104.5 63.5) (mid 104.853553 63.646447) (end 105 64) (stroke (width 0.1) (type solid)) (layer "Edge.Cuts"))
 (gr_line (start 162 44) (end 103 44) (stroke (width 0.1) (type solid)) (layer "Edge.Cuts"))
 (segment (start 118.53 48.77) (end 117.378 48.77) (width 0.2) (layer "F.Cu") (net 1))
 (segment (start 128.72 80.035) (end 129.822 80.035) (width 0.2) (layer "F.Cu") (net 1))
 (segment (start 114.602 46.23) (end 113.45 46.23) (width 0.2) (layer "F.Cu") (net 1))
 (segment (start 128.581 73.444) (end 128.864 73.7267) (width 0.2) (layer "F.Cu") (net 1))
 (segment (start 124.762 46.4985) (end 124.762 46.23) (width 0.2) (layer "F.Cu") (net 1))
 (segment (start 114.602 46.4985) (end 114.602 46.23) (width 0.2) (layer "F.Cu") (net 1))
 (segment (start 128.581 73.444) (end 127.61 74.4153) (width 0.2) (layer "F.Cu") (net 1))
 (segment (start 128.72 72.9659) (end 128.581 73.105) (width 0.2) (layer "F.Cu") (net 1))
 (segment (start 137.698 48.77) (end 137.698 48.482) (width 0.2) (layer "F.Cu") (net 1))
 (segment (start 127.61 78.0513) (end 128.492 78.9333) (width 0.2) (layer "F.Cu") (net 1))
 (segment (start 138.85 48.77) (end 137.698 48.77) (width 0.2) (layer "F.Cu") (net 1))
 (segment (start 125.684 47.4206) (end 124.762 46.4985) (width 0.2) (layer "F.Cu") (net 1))
 (segment (start 124.762 46.23) (end 123.61 46.23) (width 0.2) (layer "F.Cu") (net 1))
 (segment (start 116.515 47.6183) (end 115.722 47.6183) (width 0.2) (layer "F.Cu") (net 1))
 (segment (start 117.378 48.77) (end 117.378 48.482) (width 0.2) (layer "F.Cu") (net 1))
 (segment (start 117.378 48.482) (end 116.515 47.6183) (width 0.2) (layer "F.Cu") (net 1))
 (segment (start 130.341 47.4206) (end 125.684 47.4206) (width 0.2) (layer "F.Cu") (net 1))
 (segment (start 136.835 47.6183) (end 133.502 47.6183) (width 0.2) (layer "F.Cu") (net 1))
 (segment (start 131.23 46.23) (end 131.531 46.23) (width 0.2) (layer "F.Cu") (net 1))
 (segment (start 128.492 78.9333) (end 128.72 78.9333) (width 0.2) (layer "F.Cu") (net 1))
 (segment (start 128.581 73.105) (end 128.581 73.444) (width 0.2) (layer "F.Cu") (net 1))
 (segment (start 137.698 48.482) (end 136.835 47.6183) (width 0.2) (layer "F.Cu") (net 1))
 (segment (start 128.72 78.9333) (end 128.72 80.035) (width 0.2) (layer "F.Cu") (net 1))
 (segment (start 123.61 46.23) (end 121.07 46.23) (width 0.2) (layer "F.Cu") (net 1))
 (segment (start 133.502 47.6183) (end 132.382 46.4985) (width 0.2) (layer "F.Cu") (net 1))
 (segment (start 115.722 47.6183) (end 114.602 46.4985) (width 0.2) (layer "F.Cu") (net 1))
 (segment (start 130.357 79.5) (end 162.335 79.5) (width 0.2) (layer "F.Cu") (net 1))
 (segment (start 133.355 73.7267) (end 133.355 71.775) (width 0.2) (layer "F.Cu") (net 1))
 (segment (start 129.822 80.035) (end 130.357 79.5) (width 0.2) (layer "F.Cu") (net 1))
 (segment (start 132.382 46.23) (end 131.531 46.23) (width 0.2) (layer "F.Cu") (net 1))
 (segment (start 127.61 74.4153) (end 127.61 78.0513) (width 0.2) (layer "F.Cu") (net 1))
 (segment (start 132.382 46.4985) (end 132.382 46.23) (width 0.2) (layer "F.Cu") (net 1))
 (segment (start 128.72 72.415) (end 128.72 72.9659) (width 0.2) (layer "F.Cu") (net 1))
 (segment (start 128.864 73.7267) (end 133.355 73.7267) (width 0.2) (layer "F.Cu") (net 1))
 (segment (start 131.531 46.23) (end 130.341 47.4206) (width 0.2) (layer "F.Cu") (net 1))
 (segment (start 143.93 46.23) (end 142.778 46.23) (width 0.2) (layer "B.Cu") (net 1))
 (segment (start 133.115 67.1466) (end 133.115 61.03) (width 0.2) (layer "B.Cu") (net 1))
 (segment (start 146.004 47.4206) (end 145.082 46.4985) (width 0.2) (layer "B.Cu") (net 1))
 (segment (start 133.618 58.1783) (end 133.115 58.1783) (width 0.2) (layer "B.Cu") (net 1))
 (segment (start 140.002 48.77) (end 138.85 48.77) (width 0.2) (layer "B.Cu") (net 1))
 (segment (start 121.07 47.3817) (end 120.802 47.3817) (width 0.2) (layer "B.Cu") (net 1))
 (segment (start 141.915 47.3817) (end 141.122 47.3817) (width 0.2) (layer "B.Cu") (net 1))
 (segment (start 128.948 71.3133) (end 133.115 67.1466) (width 0.2) (layer "B.Cu") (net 1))
 (segment (start 128.72 72.415) (end 128.72 71.3133) (width 0.2) (layer "B.Cu") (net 1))
 (segment (start 138.85 52.9463) (end 133.618 58.1783) (width 0.2) (layer "B.Cu") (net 1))
 (segment (start 138.85 48.77) (end 138.85 52.9463) (width 0.2) (layer "B.Cu") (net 1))
 (segment (start 155.478 48.482) (end 154.615 47.6183) (width 0.2) (layer "B.Cu") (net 1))
 (segment (start 128.72 71.3133) (end 128.948 71.3133) (width 0.2) (layer "B.Cu") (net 1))
 (segment (start 145.082 46.23) (end 143.93 46.23) (width 0.2) (layer "B.Cu") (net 1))
 (segment (start 155.478 48.77) (end 155.478 48.482) (width 0.2) (layer "B.Cu") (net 1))
 (segment (start 119.682 48.77) (end 118.53 48.77) (width 0.2) (layer "B.Cu") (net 1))
 (segment (start 147.858 46.23) (end 147.858 46.5179) (width 0.2) (layer "B.Cu") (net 1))
 (segment (start 150.162 46.23) (end 149.01 46.23) (width 0.2) (layer "B.Cu") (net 1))
 (segment (start 146.956 47.4206) (end 146.004 47.4206) (width 0.2) (layer "B.Cu") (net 1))
 (segment (start 156.63 48.77) (end 155.478 48.77) (width 0.2) (layer "B.Cu") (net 1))
 (segment (start 140.002 48.5015) (end 140.002 48.77) (width 0.2) (layer "B.Cu") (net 1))
 (segment (start 154.615 47.6183) (end 151.282 47.6183) (width 0.2) (layer "B.Cu") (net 1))
 (segment (start 128.72 80.035) (end 128.72 82.575) (width 0.2) (layer "B.Cu") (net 1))
 (segment (start 119.682 48.5015) (end 119.682 48.77) (width 0.2) (layer "B.Cu") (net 1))
 (segment (start 151.282 47.6183) (end 150.162 46.4985) (width 0.2) (layer "B.Cu") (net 1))
 (segment (start 145.082 46.4985) (end 145.082 46.23) (width 0.2) (layer "B.Cu") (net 1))
 (segment (start 142.778 46.23) (end 142.778 46.518) (width 0.2) (layer "B.Cu") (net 1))
 (segment (start 133.115 58.1783) (end 133.115 59.03) (width 0.2) (layer "B.Cu") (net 1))
 (segment (start 120.802 47.3817) (end 119.682 48.5015) (width 0.2) (layer "B.Cu") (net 1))
 (segment (start 147.858 46.5179) (end 146.956 47.4206) (width 0.2) (layer "B.Cu") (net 1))
 (segment (start 150.162 46.4985) (end 150.162 46.23) (width 0.2) (layer "B.Cu") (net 1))
 (segment (start 121.07 46.23) (end 121.07 47.3817) (width 0.2) (layer "B.Cu") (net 1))
 (segment (start 141.122 47.3817) (end 140.002 48.5015) (width 0.2) (layer "B.Cu") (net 1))
 (segment (start 142.778 46.518) (end 141.915 47.3817) (width 0.2) (layer "B.Cu") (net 1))
 (segment (start 133.115 59.03) (end 133.115 61.03) (width 0.2) (layer "B.Cu") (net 1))
 (segment (start 149.01 46.23) (end 147.858 46.23) (width 0.2) (layer "B.Cu") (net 1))
 (segment (start 122.222 49.0234) (end 130.228 57.03) (width 0.2) (layer "F.Cu") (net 6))
 (segment (start 130.228 57.03) (end 133.115 57.03) (width 0.2) (layer "F.Cu") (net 6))
 (segment (start 122.222 48.77) (end 122.222 49.0234) (width 0.2) (layer "F.Cu") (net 6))
 (segment (start 121.07 48.77) (end 122.222 48.77) (width 0.2) (layer "F.Cu") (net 6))
 (segment (start 124.762 48.77) (end 123.61 48.77) (width 0.2) (layer "F.Cu") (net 4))
 (segment (start 162.335 77.75) (end 159.404 77.75) (width 0.2) (layer "F.Cu") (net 4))
 (segment (start 159.404 77.75) (end 137.688 56.0333) (width 0.2) (layer "F.Cu") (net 4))
 (segment (start 124.762 49.0579) (end 124.762 48.77) (width 0.2) (layer "F.Cu") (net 4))
 (segment (start 131.737 56.0333) (end 124.762 49.0579) (width 0.2) (layer "F.Cu") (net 4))
 (segment (start 137.688 56.0333) (end 131.737 56.0333) (width 0.2) (layer "F.Cu") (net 4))
 (segment (start 128.72 61.1533) (end 128.72 62.255) (width 0.2) (layer "B.Cu") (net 29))
 (segment (start 129.823 51.3285) (end 129.823 60.223) (width 0.2) (layer "B.Cu") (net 29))
 (segment (start 129.823 60.223) (end 128.893 61.1533) (width 0.2) (layer "B.Cu") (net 29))
 (segment (start 131.23 48.77) (end 131.23 49.9217) (width 0.2) (layer "B.Cu") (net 29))
 (segment (start 128.893 61.1533) (end 128.72 61.1533) (width 0.2) (layer "B.Cu") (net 29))
 (segment (start 131.23 49.9217) (end 129.823 51.3285) (width 0.2) (layer "B.Cu") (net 29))
 (segment (start 133.77 48.77) (end 133.77 51.1028) (width 0.2) (layer "B.Cu") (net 27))
 (segment (start 128.946 66.2333) (end 128.72 66.2333) (width 0.2) (layer "B.Cu") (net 27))
 (segment (start 128.72 66.2333) (end 128.72 67.335) (width 0.2) (layer "B.Cu") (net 27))
 (segment (start 130.798 64.3812) (end 128.946 66.2333) (width 0.2) (layer "B.Cu") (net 27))
 (segment (start 133.77 51.1028) (end 130.798 54.0752) (width 0.2) (layer "B.Cu") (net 27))
 (segment (start 130.798 54.0752) (end 130.798 64.3812) (width 0.2) (layer "B.Cu") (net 27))
 (segment (start 128.72 68.7733) (end 128.72 69.875) (width 0.2) (layer "B.Cu") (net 26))
 (segment (start 129.96 49.2176) (end 127.615 51.5622) (width 0.2) (layer "B.Cu") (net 26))
 (segment (start 130.963 47.3817) (end 129.96 48.3846) (width 0.2) (layer "B.Cu") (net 26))
 (segment (start 128.492 68.7733) (end 128.72 68.7733) (width 0.2) (layer "B.Cu") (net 26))
 (segment (start 132.618 46.518) (end 131.755 47.3817) (width 0.2) (layer "B.Cu") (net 26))
 (segment (start 127.615 67.897) (end 128.492 68.7733) (width 0.2) (layer "B.Cu") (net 26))
 (segment (start 127.615 51.5622) (end 127.615 67.897) (width 0.2) (layer "B.Cu") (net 26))
 (segment (start 129.96 48.3846) (end 129.96 49.2176) (width 0.2) (layer "B.Cu") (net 26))
 (segment (start 133.77 46.23) (end 132.618 46.23) (width 0.2) (layer "B.Cu") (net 26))
 (segment (start 131.755 47.3817) (end 130.963 47.3817) (width 0.2) (layer "B.Cu") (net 26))
 (segment (start 132.618 46.23) (end 132.618 46.518) (width 0.2) (layer "B.Cu") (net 26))
 (segment (start 132.441 51.722) (end 130.249 53.9143) (width 0.2) (layer "B.Cu") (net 28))
 (segment (start 134.289 47.613) (end 133.239 47.613) (width 0.2) (layer "B.Cu") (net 28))
 (segment (start 128.72 63.6933) (end 128.72 64.795) (width 0.2) (layer "B.Cu") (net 28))
 (segment (start 128.948 63.6933) (end 128.72 63.6933) (width 0.2) (layer "B.Cu") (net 28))
 (segment (start 135.158 48.4821) (end 134.289 47.613) (width 0.2) (layer "B.Cu") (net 28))
 (segment (start 135.158 48.77) (end 135.158 48.4821) (width 0.2) (layer "B.Cu") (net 28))
 (segment (start 136.31 48.77) (end 135.158 48.77) (width 0.2) (layer "B.Cu") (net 28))
 (segment (start 133.239 47.613) (end 132.441 48.4102) (width 0.2) (layer "B.Cu") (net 28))
 (segment (start 130.249 53.9143) (end 130.249 62.3925) (width 0.2) (layer "B.Cu") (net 28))
 (segment (start 130.249 62.3925) (end 128.948 63.6933) (width 0.2) (layer "B.Cu") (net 28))
 (segment (start 132.441 48.4102) (end 132.441 51.722) (width 0.2) (layer "B.Cu") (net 28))
 (segment (start 128.72 59.715) (end 128.169 59.715) (width 0.2) (layer "F.Cu") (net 2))
 (segment (start 110.91 46.8058) (end 110.098 46.8058) (width 0.2) (layer "F.Cu") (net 2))
 (segment (start 131.905 73.025) (end 131.253 73.025) (width 0.2) (layer "F.Cu") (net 2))
 (segment (start 110.91 47.3817) (end 111.198 47.3817) (width 0.2) (layer "F.Cu") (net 2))
 (segment (start 110.91 46.8058) (end 110.91 47.3817) (width 0.2) (layer "F.Cu") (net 2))
 (segment (start 131.253 73.025) (end 131.253 70.2632) (width 0.2) (layer "F.Cu") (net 2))
 (segment (start 91.61 61.435) (end 91.61 53.931492) (width 0.2) (layer "F.Cu") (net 2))
 (segment (start 131.253 70.2632) (end 131.693 69.8233) (width 0.2) (layer "F.Cu") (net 2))
 (segment (start 101.691492 43.85) (end 107 43.85) (width 0.2) (layer "F.Cu") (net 2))
 (segment (start 123.088 55.1845) (end 127.618 59.715) (width 0.2) (layer "F.Cu") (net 2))
 (segment (start 131.693 63.239) (end 131.693 69.8233) (width 0.2) (layer "F.Cu") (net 2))
 (segment (start 101.691492 43.85) (end 119 43.85) (width 0.2) (layer "F.Cu") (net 2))
 (segment (start 131.693 69.8233) (end 135.05 69.8233) (width 0.2) (layer "F.Cu") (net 2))
 (segment (start 111.198 47.3817) (end 112.062 48.2454) (width 0.2) (layer "F.Cu") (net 2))
 (segment (start 135.05 69.8233) (end 135.457 70.2305) (width 0.2) (layer "F.Cu") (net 2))
 (segment (start 101.691492 43.85) (end 108.5 43.85) (width 0.2) (layer "F.Cu") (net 2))
 (segment (start 110.91 46.23) (end 110.91 46.8058) (width 0.2) (layer "F.Cu") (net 2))
 (segment (start 118.199 55.1845) (end 123.088 55.1845) (width 0.2) (layer "F.Cu") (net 2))
 (segment (start 112.062 48.2454) (end 112.062 49.0475) (width 0.2) (layer "F.Cu") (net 2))
 (segment (start 91.61 53.931492) (end 101.691492 43.85) (width 0.2) (layer "F.Cu") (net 2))
 (segment (start 128.169 59.715) (end 131.693 63.239) (width 0.2) (layer "F.Cu") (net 2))
 (segment (start 127.618 59.715) (end 128.169 59.715) (width 0.2) (layer "F.Cu") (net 2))
 (segment (start 135.457 70.2305) (end 135.457 70.525) (width 0.2) (layer "F.Cu") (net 2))
 (segment (start 135.457 70.525) (end 134.805 70.525) (width 0.2) (layer "F.Cu") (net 2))
 (segment (start 91.61 80.565) (end 91.61 53.931492) (width 0.2) (layer "F.Cu") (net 2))
 (segment (start 110.098 46.8058) (end 109.522 46.23) (width 0.2) (layer "F.Cu") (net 2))
 (segment (start 109.522 46.23) (end 108.37 46.23) (width 0.2) (layer "F.Cu") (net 2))
 (segment (start 112.062 49.0475) (end 118.199 55.1845) (width 0.2) (layer "F.Cu") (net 2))
 (segment (start 108.37 48.77) (end 109.522 48.77) (width 0.2) (layer "B.Cu") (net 25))
 (segment (start 126.674 72.0361) (end 128.492 73.8533) (width 0.2) (layer "B.Cu") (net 25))
 (segment (start 126.674 49.9217) (end 126.674 72.0361) (width 0.2) (layer "B.Cu") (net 25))
 (segment (start 110.385 49.9217) (end 126.674 49.9217) (width 0.2) (layer "B.Cu") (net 25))
 (segment (start 127.538 48.77) (end 127.538 49.0579) (width 0.2) (layer "B.Cu") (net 25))
 (segment (start 128.72 73.8533) (end 128.72 74.955) (width 0.2) (layer "B.Cu") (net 25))
 (segment (start 109.522 48.77) (end 109.522 49.058) (width 0.2) (layer "B.Cu") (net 25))
 (segment (start 127.538 49.0579) (end 126.674 49.9217) (width 0.2) (layer "B.Cu") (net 25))
 (segment (start 109.522 49.058) (end 110.385 49.9217) (width 0.2) (layer "B.Cu") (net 25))
 (segment (start 128.492 73.8533) (end 128.72 73.8533) (width 0.2) (layer "B.Cu") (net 25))
 (segment (start 128.69 48.77) (end 127.538 48.77) (width 0.2) (layer "B.Cu") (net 25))
 (segment (start 145.799 60.3) (end 162.975 77.4759) (width 0.2) (layer "F.Cu") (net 5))
 (segment (start 162.975 77.4759) (end 162.975 77.75) (width 0.2) (layer "F.Cu") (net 5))
 (segment (start 143.415 60.3) (end 145.799 60.3) (width 0.2) (layer "F.Cu") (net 5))
 (segment (start 128.72 77.495) (end 129.822 77.495) (width 0.2) (layer "F.Cu") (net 3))
 (segment (start 162.975 79.3201) (end 162.975 79.5) (width 0.2) (layer "F.Cu") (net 3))
 (segment (start 129.822 77.495) (end 130.923 78.5967) (width 0.2) (layer "F.Cu") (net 3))
 (segment (start 130.923 78.5967) (end 162.252 78.5967) (width 0.2) (layer "F.Cu") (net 3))
 (segment (start 162.252 78.5967) (end 162.975 79.3201) (width 0.2) (layer "F.Cu") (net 3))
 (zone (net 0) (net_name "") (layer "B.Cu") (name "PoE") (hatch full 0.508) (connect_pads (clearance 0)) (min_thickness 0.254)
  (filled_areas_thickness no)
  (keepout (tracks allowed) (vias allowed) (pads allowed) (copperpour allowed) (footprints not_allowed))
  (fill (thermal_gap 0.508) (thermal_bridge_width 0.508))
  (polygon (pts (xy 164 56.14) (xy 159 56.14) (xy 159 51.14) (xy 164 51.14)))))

